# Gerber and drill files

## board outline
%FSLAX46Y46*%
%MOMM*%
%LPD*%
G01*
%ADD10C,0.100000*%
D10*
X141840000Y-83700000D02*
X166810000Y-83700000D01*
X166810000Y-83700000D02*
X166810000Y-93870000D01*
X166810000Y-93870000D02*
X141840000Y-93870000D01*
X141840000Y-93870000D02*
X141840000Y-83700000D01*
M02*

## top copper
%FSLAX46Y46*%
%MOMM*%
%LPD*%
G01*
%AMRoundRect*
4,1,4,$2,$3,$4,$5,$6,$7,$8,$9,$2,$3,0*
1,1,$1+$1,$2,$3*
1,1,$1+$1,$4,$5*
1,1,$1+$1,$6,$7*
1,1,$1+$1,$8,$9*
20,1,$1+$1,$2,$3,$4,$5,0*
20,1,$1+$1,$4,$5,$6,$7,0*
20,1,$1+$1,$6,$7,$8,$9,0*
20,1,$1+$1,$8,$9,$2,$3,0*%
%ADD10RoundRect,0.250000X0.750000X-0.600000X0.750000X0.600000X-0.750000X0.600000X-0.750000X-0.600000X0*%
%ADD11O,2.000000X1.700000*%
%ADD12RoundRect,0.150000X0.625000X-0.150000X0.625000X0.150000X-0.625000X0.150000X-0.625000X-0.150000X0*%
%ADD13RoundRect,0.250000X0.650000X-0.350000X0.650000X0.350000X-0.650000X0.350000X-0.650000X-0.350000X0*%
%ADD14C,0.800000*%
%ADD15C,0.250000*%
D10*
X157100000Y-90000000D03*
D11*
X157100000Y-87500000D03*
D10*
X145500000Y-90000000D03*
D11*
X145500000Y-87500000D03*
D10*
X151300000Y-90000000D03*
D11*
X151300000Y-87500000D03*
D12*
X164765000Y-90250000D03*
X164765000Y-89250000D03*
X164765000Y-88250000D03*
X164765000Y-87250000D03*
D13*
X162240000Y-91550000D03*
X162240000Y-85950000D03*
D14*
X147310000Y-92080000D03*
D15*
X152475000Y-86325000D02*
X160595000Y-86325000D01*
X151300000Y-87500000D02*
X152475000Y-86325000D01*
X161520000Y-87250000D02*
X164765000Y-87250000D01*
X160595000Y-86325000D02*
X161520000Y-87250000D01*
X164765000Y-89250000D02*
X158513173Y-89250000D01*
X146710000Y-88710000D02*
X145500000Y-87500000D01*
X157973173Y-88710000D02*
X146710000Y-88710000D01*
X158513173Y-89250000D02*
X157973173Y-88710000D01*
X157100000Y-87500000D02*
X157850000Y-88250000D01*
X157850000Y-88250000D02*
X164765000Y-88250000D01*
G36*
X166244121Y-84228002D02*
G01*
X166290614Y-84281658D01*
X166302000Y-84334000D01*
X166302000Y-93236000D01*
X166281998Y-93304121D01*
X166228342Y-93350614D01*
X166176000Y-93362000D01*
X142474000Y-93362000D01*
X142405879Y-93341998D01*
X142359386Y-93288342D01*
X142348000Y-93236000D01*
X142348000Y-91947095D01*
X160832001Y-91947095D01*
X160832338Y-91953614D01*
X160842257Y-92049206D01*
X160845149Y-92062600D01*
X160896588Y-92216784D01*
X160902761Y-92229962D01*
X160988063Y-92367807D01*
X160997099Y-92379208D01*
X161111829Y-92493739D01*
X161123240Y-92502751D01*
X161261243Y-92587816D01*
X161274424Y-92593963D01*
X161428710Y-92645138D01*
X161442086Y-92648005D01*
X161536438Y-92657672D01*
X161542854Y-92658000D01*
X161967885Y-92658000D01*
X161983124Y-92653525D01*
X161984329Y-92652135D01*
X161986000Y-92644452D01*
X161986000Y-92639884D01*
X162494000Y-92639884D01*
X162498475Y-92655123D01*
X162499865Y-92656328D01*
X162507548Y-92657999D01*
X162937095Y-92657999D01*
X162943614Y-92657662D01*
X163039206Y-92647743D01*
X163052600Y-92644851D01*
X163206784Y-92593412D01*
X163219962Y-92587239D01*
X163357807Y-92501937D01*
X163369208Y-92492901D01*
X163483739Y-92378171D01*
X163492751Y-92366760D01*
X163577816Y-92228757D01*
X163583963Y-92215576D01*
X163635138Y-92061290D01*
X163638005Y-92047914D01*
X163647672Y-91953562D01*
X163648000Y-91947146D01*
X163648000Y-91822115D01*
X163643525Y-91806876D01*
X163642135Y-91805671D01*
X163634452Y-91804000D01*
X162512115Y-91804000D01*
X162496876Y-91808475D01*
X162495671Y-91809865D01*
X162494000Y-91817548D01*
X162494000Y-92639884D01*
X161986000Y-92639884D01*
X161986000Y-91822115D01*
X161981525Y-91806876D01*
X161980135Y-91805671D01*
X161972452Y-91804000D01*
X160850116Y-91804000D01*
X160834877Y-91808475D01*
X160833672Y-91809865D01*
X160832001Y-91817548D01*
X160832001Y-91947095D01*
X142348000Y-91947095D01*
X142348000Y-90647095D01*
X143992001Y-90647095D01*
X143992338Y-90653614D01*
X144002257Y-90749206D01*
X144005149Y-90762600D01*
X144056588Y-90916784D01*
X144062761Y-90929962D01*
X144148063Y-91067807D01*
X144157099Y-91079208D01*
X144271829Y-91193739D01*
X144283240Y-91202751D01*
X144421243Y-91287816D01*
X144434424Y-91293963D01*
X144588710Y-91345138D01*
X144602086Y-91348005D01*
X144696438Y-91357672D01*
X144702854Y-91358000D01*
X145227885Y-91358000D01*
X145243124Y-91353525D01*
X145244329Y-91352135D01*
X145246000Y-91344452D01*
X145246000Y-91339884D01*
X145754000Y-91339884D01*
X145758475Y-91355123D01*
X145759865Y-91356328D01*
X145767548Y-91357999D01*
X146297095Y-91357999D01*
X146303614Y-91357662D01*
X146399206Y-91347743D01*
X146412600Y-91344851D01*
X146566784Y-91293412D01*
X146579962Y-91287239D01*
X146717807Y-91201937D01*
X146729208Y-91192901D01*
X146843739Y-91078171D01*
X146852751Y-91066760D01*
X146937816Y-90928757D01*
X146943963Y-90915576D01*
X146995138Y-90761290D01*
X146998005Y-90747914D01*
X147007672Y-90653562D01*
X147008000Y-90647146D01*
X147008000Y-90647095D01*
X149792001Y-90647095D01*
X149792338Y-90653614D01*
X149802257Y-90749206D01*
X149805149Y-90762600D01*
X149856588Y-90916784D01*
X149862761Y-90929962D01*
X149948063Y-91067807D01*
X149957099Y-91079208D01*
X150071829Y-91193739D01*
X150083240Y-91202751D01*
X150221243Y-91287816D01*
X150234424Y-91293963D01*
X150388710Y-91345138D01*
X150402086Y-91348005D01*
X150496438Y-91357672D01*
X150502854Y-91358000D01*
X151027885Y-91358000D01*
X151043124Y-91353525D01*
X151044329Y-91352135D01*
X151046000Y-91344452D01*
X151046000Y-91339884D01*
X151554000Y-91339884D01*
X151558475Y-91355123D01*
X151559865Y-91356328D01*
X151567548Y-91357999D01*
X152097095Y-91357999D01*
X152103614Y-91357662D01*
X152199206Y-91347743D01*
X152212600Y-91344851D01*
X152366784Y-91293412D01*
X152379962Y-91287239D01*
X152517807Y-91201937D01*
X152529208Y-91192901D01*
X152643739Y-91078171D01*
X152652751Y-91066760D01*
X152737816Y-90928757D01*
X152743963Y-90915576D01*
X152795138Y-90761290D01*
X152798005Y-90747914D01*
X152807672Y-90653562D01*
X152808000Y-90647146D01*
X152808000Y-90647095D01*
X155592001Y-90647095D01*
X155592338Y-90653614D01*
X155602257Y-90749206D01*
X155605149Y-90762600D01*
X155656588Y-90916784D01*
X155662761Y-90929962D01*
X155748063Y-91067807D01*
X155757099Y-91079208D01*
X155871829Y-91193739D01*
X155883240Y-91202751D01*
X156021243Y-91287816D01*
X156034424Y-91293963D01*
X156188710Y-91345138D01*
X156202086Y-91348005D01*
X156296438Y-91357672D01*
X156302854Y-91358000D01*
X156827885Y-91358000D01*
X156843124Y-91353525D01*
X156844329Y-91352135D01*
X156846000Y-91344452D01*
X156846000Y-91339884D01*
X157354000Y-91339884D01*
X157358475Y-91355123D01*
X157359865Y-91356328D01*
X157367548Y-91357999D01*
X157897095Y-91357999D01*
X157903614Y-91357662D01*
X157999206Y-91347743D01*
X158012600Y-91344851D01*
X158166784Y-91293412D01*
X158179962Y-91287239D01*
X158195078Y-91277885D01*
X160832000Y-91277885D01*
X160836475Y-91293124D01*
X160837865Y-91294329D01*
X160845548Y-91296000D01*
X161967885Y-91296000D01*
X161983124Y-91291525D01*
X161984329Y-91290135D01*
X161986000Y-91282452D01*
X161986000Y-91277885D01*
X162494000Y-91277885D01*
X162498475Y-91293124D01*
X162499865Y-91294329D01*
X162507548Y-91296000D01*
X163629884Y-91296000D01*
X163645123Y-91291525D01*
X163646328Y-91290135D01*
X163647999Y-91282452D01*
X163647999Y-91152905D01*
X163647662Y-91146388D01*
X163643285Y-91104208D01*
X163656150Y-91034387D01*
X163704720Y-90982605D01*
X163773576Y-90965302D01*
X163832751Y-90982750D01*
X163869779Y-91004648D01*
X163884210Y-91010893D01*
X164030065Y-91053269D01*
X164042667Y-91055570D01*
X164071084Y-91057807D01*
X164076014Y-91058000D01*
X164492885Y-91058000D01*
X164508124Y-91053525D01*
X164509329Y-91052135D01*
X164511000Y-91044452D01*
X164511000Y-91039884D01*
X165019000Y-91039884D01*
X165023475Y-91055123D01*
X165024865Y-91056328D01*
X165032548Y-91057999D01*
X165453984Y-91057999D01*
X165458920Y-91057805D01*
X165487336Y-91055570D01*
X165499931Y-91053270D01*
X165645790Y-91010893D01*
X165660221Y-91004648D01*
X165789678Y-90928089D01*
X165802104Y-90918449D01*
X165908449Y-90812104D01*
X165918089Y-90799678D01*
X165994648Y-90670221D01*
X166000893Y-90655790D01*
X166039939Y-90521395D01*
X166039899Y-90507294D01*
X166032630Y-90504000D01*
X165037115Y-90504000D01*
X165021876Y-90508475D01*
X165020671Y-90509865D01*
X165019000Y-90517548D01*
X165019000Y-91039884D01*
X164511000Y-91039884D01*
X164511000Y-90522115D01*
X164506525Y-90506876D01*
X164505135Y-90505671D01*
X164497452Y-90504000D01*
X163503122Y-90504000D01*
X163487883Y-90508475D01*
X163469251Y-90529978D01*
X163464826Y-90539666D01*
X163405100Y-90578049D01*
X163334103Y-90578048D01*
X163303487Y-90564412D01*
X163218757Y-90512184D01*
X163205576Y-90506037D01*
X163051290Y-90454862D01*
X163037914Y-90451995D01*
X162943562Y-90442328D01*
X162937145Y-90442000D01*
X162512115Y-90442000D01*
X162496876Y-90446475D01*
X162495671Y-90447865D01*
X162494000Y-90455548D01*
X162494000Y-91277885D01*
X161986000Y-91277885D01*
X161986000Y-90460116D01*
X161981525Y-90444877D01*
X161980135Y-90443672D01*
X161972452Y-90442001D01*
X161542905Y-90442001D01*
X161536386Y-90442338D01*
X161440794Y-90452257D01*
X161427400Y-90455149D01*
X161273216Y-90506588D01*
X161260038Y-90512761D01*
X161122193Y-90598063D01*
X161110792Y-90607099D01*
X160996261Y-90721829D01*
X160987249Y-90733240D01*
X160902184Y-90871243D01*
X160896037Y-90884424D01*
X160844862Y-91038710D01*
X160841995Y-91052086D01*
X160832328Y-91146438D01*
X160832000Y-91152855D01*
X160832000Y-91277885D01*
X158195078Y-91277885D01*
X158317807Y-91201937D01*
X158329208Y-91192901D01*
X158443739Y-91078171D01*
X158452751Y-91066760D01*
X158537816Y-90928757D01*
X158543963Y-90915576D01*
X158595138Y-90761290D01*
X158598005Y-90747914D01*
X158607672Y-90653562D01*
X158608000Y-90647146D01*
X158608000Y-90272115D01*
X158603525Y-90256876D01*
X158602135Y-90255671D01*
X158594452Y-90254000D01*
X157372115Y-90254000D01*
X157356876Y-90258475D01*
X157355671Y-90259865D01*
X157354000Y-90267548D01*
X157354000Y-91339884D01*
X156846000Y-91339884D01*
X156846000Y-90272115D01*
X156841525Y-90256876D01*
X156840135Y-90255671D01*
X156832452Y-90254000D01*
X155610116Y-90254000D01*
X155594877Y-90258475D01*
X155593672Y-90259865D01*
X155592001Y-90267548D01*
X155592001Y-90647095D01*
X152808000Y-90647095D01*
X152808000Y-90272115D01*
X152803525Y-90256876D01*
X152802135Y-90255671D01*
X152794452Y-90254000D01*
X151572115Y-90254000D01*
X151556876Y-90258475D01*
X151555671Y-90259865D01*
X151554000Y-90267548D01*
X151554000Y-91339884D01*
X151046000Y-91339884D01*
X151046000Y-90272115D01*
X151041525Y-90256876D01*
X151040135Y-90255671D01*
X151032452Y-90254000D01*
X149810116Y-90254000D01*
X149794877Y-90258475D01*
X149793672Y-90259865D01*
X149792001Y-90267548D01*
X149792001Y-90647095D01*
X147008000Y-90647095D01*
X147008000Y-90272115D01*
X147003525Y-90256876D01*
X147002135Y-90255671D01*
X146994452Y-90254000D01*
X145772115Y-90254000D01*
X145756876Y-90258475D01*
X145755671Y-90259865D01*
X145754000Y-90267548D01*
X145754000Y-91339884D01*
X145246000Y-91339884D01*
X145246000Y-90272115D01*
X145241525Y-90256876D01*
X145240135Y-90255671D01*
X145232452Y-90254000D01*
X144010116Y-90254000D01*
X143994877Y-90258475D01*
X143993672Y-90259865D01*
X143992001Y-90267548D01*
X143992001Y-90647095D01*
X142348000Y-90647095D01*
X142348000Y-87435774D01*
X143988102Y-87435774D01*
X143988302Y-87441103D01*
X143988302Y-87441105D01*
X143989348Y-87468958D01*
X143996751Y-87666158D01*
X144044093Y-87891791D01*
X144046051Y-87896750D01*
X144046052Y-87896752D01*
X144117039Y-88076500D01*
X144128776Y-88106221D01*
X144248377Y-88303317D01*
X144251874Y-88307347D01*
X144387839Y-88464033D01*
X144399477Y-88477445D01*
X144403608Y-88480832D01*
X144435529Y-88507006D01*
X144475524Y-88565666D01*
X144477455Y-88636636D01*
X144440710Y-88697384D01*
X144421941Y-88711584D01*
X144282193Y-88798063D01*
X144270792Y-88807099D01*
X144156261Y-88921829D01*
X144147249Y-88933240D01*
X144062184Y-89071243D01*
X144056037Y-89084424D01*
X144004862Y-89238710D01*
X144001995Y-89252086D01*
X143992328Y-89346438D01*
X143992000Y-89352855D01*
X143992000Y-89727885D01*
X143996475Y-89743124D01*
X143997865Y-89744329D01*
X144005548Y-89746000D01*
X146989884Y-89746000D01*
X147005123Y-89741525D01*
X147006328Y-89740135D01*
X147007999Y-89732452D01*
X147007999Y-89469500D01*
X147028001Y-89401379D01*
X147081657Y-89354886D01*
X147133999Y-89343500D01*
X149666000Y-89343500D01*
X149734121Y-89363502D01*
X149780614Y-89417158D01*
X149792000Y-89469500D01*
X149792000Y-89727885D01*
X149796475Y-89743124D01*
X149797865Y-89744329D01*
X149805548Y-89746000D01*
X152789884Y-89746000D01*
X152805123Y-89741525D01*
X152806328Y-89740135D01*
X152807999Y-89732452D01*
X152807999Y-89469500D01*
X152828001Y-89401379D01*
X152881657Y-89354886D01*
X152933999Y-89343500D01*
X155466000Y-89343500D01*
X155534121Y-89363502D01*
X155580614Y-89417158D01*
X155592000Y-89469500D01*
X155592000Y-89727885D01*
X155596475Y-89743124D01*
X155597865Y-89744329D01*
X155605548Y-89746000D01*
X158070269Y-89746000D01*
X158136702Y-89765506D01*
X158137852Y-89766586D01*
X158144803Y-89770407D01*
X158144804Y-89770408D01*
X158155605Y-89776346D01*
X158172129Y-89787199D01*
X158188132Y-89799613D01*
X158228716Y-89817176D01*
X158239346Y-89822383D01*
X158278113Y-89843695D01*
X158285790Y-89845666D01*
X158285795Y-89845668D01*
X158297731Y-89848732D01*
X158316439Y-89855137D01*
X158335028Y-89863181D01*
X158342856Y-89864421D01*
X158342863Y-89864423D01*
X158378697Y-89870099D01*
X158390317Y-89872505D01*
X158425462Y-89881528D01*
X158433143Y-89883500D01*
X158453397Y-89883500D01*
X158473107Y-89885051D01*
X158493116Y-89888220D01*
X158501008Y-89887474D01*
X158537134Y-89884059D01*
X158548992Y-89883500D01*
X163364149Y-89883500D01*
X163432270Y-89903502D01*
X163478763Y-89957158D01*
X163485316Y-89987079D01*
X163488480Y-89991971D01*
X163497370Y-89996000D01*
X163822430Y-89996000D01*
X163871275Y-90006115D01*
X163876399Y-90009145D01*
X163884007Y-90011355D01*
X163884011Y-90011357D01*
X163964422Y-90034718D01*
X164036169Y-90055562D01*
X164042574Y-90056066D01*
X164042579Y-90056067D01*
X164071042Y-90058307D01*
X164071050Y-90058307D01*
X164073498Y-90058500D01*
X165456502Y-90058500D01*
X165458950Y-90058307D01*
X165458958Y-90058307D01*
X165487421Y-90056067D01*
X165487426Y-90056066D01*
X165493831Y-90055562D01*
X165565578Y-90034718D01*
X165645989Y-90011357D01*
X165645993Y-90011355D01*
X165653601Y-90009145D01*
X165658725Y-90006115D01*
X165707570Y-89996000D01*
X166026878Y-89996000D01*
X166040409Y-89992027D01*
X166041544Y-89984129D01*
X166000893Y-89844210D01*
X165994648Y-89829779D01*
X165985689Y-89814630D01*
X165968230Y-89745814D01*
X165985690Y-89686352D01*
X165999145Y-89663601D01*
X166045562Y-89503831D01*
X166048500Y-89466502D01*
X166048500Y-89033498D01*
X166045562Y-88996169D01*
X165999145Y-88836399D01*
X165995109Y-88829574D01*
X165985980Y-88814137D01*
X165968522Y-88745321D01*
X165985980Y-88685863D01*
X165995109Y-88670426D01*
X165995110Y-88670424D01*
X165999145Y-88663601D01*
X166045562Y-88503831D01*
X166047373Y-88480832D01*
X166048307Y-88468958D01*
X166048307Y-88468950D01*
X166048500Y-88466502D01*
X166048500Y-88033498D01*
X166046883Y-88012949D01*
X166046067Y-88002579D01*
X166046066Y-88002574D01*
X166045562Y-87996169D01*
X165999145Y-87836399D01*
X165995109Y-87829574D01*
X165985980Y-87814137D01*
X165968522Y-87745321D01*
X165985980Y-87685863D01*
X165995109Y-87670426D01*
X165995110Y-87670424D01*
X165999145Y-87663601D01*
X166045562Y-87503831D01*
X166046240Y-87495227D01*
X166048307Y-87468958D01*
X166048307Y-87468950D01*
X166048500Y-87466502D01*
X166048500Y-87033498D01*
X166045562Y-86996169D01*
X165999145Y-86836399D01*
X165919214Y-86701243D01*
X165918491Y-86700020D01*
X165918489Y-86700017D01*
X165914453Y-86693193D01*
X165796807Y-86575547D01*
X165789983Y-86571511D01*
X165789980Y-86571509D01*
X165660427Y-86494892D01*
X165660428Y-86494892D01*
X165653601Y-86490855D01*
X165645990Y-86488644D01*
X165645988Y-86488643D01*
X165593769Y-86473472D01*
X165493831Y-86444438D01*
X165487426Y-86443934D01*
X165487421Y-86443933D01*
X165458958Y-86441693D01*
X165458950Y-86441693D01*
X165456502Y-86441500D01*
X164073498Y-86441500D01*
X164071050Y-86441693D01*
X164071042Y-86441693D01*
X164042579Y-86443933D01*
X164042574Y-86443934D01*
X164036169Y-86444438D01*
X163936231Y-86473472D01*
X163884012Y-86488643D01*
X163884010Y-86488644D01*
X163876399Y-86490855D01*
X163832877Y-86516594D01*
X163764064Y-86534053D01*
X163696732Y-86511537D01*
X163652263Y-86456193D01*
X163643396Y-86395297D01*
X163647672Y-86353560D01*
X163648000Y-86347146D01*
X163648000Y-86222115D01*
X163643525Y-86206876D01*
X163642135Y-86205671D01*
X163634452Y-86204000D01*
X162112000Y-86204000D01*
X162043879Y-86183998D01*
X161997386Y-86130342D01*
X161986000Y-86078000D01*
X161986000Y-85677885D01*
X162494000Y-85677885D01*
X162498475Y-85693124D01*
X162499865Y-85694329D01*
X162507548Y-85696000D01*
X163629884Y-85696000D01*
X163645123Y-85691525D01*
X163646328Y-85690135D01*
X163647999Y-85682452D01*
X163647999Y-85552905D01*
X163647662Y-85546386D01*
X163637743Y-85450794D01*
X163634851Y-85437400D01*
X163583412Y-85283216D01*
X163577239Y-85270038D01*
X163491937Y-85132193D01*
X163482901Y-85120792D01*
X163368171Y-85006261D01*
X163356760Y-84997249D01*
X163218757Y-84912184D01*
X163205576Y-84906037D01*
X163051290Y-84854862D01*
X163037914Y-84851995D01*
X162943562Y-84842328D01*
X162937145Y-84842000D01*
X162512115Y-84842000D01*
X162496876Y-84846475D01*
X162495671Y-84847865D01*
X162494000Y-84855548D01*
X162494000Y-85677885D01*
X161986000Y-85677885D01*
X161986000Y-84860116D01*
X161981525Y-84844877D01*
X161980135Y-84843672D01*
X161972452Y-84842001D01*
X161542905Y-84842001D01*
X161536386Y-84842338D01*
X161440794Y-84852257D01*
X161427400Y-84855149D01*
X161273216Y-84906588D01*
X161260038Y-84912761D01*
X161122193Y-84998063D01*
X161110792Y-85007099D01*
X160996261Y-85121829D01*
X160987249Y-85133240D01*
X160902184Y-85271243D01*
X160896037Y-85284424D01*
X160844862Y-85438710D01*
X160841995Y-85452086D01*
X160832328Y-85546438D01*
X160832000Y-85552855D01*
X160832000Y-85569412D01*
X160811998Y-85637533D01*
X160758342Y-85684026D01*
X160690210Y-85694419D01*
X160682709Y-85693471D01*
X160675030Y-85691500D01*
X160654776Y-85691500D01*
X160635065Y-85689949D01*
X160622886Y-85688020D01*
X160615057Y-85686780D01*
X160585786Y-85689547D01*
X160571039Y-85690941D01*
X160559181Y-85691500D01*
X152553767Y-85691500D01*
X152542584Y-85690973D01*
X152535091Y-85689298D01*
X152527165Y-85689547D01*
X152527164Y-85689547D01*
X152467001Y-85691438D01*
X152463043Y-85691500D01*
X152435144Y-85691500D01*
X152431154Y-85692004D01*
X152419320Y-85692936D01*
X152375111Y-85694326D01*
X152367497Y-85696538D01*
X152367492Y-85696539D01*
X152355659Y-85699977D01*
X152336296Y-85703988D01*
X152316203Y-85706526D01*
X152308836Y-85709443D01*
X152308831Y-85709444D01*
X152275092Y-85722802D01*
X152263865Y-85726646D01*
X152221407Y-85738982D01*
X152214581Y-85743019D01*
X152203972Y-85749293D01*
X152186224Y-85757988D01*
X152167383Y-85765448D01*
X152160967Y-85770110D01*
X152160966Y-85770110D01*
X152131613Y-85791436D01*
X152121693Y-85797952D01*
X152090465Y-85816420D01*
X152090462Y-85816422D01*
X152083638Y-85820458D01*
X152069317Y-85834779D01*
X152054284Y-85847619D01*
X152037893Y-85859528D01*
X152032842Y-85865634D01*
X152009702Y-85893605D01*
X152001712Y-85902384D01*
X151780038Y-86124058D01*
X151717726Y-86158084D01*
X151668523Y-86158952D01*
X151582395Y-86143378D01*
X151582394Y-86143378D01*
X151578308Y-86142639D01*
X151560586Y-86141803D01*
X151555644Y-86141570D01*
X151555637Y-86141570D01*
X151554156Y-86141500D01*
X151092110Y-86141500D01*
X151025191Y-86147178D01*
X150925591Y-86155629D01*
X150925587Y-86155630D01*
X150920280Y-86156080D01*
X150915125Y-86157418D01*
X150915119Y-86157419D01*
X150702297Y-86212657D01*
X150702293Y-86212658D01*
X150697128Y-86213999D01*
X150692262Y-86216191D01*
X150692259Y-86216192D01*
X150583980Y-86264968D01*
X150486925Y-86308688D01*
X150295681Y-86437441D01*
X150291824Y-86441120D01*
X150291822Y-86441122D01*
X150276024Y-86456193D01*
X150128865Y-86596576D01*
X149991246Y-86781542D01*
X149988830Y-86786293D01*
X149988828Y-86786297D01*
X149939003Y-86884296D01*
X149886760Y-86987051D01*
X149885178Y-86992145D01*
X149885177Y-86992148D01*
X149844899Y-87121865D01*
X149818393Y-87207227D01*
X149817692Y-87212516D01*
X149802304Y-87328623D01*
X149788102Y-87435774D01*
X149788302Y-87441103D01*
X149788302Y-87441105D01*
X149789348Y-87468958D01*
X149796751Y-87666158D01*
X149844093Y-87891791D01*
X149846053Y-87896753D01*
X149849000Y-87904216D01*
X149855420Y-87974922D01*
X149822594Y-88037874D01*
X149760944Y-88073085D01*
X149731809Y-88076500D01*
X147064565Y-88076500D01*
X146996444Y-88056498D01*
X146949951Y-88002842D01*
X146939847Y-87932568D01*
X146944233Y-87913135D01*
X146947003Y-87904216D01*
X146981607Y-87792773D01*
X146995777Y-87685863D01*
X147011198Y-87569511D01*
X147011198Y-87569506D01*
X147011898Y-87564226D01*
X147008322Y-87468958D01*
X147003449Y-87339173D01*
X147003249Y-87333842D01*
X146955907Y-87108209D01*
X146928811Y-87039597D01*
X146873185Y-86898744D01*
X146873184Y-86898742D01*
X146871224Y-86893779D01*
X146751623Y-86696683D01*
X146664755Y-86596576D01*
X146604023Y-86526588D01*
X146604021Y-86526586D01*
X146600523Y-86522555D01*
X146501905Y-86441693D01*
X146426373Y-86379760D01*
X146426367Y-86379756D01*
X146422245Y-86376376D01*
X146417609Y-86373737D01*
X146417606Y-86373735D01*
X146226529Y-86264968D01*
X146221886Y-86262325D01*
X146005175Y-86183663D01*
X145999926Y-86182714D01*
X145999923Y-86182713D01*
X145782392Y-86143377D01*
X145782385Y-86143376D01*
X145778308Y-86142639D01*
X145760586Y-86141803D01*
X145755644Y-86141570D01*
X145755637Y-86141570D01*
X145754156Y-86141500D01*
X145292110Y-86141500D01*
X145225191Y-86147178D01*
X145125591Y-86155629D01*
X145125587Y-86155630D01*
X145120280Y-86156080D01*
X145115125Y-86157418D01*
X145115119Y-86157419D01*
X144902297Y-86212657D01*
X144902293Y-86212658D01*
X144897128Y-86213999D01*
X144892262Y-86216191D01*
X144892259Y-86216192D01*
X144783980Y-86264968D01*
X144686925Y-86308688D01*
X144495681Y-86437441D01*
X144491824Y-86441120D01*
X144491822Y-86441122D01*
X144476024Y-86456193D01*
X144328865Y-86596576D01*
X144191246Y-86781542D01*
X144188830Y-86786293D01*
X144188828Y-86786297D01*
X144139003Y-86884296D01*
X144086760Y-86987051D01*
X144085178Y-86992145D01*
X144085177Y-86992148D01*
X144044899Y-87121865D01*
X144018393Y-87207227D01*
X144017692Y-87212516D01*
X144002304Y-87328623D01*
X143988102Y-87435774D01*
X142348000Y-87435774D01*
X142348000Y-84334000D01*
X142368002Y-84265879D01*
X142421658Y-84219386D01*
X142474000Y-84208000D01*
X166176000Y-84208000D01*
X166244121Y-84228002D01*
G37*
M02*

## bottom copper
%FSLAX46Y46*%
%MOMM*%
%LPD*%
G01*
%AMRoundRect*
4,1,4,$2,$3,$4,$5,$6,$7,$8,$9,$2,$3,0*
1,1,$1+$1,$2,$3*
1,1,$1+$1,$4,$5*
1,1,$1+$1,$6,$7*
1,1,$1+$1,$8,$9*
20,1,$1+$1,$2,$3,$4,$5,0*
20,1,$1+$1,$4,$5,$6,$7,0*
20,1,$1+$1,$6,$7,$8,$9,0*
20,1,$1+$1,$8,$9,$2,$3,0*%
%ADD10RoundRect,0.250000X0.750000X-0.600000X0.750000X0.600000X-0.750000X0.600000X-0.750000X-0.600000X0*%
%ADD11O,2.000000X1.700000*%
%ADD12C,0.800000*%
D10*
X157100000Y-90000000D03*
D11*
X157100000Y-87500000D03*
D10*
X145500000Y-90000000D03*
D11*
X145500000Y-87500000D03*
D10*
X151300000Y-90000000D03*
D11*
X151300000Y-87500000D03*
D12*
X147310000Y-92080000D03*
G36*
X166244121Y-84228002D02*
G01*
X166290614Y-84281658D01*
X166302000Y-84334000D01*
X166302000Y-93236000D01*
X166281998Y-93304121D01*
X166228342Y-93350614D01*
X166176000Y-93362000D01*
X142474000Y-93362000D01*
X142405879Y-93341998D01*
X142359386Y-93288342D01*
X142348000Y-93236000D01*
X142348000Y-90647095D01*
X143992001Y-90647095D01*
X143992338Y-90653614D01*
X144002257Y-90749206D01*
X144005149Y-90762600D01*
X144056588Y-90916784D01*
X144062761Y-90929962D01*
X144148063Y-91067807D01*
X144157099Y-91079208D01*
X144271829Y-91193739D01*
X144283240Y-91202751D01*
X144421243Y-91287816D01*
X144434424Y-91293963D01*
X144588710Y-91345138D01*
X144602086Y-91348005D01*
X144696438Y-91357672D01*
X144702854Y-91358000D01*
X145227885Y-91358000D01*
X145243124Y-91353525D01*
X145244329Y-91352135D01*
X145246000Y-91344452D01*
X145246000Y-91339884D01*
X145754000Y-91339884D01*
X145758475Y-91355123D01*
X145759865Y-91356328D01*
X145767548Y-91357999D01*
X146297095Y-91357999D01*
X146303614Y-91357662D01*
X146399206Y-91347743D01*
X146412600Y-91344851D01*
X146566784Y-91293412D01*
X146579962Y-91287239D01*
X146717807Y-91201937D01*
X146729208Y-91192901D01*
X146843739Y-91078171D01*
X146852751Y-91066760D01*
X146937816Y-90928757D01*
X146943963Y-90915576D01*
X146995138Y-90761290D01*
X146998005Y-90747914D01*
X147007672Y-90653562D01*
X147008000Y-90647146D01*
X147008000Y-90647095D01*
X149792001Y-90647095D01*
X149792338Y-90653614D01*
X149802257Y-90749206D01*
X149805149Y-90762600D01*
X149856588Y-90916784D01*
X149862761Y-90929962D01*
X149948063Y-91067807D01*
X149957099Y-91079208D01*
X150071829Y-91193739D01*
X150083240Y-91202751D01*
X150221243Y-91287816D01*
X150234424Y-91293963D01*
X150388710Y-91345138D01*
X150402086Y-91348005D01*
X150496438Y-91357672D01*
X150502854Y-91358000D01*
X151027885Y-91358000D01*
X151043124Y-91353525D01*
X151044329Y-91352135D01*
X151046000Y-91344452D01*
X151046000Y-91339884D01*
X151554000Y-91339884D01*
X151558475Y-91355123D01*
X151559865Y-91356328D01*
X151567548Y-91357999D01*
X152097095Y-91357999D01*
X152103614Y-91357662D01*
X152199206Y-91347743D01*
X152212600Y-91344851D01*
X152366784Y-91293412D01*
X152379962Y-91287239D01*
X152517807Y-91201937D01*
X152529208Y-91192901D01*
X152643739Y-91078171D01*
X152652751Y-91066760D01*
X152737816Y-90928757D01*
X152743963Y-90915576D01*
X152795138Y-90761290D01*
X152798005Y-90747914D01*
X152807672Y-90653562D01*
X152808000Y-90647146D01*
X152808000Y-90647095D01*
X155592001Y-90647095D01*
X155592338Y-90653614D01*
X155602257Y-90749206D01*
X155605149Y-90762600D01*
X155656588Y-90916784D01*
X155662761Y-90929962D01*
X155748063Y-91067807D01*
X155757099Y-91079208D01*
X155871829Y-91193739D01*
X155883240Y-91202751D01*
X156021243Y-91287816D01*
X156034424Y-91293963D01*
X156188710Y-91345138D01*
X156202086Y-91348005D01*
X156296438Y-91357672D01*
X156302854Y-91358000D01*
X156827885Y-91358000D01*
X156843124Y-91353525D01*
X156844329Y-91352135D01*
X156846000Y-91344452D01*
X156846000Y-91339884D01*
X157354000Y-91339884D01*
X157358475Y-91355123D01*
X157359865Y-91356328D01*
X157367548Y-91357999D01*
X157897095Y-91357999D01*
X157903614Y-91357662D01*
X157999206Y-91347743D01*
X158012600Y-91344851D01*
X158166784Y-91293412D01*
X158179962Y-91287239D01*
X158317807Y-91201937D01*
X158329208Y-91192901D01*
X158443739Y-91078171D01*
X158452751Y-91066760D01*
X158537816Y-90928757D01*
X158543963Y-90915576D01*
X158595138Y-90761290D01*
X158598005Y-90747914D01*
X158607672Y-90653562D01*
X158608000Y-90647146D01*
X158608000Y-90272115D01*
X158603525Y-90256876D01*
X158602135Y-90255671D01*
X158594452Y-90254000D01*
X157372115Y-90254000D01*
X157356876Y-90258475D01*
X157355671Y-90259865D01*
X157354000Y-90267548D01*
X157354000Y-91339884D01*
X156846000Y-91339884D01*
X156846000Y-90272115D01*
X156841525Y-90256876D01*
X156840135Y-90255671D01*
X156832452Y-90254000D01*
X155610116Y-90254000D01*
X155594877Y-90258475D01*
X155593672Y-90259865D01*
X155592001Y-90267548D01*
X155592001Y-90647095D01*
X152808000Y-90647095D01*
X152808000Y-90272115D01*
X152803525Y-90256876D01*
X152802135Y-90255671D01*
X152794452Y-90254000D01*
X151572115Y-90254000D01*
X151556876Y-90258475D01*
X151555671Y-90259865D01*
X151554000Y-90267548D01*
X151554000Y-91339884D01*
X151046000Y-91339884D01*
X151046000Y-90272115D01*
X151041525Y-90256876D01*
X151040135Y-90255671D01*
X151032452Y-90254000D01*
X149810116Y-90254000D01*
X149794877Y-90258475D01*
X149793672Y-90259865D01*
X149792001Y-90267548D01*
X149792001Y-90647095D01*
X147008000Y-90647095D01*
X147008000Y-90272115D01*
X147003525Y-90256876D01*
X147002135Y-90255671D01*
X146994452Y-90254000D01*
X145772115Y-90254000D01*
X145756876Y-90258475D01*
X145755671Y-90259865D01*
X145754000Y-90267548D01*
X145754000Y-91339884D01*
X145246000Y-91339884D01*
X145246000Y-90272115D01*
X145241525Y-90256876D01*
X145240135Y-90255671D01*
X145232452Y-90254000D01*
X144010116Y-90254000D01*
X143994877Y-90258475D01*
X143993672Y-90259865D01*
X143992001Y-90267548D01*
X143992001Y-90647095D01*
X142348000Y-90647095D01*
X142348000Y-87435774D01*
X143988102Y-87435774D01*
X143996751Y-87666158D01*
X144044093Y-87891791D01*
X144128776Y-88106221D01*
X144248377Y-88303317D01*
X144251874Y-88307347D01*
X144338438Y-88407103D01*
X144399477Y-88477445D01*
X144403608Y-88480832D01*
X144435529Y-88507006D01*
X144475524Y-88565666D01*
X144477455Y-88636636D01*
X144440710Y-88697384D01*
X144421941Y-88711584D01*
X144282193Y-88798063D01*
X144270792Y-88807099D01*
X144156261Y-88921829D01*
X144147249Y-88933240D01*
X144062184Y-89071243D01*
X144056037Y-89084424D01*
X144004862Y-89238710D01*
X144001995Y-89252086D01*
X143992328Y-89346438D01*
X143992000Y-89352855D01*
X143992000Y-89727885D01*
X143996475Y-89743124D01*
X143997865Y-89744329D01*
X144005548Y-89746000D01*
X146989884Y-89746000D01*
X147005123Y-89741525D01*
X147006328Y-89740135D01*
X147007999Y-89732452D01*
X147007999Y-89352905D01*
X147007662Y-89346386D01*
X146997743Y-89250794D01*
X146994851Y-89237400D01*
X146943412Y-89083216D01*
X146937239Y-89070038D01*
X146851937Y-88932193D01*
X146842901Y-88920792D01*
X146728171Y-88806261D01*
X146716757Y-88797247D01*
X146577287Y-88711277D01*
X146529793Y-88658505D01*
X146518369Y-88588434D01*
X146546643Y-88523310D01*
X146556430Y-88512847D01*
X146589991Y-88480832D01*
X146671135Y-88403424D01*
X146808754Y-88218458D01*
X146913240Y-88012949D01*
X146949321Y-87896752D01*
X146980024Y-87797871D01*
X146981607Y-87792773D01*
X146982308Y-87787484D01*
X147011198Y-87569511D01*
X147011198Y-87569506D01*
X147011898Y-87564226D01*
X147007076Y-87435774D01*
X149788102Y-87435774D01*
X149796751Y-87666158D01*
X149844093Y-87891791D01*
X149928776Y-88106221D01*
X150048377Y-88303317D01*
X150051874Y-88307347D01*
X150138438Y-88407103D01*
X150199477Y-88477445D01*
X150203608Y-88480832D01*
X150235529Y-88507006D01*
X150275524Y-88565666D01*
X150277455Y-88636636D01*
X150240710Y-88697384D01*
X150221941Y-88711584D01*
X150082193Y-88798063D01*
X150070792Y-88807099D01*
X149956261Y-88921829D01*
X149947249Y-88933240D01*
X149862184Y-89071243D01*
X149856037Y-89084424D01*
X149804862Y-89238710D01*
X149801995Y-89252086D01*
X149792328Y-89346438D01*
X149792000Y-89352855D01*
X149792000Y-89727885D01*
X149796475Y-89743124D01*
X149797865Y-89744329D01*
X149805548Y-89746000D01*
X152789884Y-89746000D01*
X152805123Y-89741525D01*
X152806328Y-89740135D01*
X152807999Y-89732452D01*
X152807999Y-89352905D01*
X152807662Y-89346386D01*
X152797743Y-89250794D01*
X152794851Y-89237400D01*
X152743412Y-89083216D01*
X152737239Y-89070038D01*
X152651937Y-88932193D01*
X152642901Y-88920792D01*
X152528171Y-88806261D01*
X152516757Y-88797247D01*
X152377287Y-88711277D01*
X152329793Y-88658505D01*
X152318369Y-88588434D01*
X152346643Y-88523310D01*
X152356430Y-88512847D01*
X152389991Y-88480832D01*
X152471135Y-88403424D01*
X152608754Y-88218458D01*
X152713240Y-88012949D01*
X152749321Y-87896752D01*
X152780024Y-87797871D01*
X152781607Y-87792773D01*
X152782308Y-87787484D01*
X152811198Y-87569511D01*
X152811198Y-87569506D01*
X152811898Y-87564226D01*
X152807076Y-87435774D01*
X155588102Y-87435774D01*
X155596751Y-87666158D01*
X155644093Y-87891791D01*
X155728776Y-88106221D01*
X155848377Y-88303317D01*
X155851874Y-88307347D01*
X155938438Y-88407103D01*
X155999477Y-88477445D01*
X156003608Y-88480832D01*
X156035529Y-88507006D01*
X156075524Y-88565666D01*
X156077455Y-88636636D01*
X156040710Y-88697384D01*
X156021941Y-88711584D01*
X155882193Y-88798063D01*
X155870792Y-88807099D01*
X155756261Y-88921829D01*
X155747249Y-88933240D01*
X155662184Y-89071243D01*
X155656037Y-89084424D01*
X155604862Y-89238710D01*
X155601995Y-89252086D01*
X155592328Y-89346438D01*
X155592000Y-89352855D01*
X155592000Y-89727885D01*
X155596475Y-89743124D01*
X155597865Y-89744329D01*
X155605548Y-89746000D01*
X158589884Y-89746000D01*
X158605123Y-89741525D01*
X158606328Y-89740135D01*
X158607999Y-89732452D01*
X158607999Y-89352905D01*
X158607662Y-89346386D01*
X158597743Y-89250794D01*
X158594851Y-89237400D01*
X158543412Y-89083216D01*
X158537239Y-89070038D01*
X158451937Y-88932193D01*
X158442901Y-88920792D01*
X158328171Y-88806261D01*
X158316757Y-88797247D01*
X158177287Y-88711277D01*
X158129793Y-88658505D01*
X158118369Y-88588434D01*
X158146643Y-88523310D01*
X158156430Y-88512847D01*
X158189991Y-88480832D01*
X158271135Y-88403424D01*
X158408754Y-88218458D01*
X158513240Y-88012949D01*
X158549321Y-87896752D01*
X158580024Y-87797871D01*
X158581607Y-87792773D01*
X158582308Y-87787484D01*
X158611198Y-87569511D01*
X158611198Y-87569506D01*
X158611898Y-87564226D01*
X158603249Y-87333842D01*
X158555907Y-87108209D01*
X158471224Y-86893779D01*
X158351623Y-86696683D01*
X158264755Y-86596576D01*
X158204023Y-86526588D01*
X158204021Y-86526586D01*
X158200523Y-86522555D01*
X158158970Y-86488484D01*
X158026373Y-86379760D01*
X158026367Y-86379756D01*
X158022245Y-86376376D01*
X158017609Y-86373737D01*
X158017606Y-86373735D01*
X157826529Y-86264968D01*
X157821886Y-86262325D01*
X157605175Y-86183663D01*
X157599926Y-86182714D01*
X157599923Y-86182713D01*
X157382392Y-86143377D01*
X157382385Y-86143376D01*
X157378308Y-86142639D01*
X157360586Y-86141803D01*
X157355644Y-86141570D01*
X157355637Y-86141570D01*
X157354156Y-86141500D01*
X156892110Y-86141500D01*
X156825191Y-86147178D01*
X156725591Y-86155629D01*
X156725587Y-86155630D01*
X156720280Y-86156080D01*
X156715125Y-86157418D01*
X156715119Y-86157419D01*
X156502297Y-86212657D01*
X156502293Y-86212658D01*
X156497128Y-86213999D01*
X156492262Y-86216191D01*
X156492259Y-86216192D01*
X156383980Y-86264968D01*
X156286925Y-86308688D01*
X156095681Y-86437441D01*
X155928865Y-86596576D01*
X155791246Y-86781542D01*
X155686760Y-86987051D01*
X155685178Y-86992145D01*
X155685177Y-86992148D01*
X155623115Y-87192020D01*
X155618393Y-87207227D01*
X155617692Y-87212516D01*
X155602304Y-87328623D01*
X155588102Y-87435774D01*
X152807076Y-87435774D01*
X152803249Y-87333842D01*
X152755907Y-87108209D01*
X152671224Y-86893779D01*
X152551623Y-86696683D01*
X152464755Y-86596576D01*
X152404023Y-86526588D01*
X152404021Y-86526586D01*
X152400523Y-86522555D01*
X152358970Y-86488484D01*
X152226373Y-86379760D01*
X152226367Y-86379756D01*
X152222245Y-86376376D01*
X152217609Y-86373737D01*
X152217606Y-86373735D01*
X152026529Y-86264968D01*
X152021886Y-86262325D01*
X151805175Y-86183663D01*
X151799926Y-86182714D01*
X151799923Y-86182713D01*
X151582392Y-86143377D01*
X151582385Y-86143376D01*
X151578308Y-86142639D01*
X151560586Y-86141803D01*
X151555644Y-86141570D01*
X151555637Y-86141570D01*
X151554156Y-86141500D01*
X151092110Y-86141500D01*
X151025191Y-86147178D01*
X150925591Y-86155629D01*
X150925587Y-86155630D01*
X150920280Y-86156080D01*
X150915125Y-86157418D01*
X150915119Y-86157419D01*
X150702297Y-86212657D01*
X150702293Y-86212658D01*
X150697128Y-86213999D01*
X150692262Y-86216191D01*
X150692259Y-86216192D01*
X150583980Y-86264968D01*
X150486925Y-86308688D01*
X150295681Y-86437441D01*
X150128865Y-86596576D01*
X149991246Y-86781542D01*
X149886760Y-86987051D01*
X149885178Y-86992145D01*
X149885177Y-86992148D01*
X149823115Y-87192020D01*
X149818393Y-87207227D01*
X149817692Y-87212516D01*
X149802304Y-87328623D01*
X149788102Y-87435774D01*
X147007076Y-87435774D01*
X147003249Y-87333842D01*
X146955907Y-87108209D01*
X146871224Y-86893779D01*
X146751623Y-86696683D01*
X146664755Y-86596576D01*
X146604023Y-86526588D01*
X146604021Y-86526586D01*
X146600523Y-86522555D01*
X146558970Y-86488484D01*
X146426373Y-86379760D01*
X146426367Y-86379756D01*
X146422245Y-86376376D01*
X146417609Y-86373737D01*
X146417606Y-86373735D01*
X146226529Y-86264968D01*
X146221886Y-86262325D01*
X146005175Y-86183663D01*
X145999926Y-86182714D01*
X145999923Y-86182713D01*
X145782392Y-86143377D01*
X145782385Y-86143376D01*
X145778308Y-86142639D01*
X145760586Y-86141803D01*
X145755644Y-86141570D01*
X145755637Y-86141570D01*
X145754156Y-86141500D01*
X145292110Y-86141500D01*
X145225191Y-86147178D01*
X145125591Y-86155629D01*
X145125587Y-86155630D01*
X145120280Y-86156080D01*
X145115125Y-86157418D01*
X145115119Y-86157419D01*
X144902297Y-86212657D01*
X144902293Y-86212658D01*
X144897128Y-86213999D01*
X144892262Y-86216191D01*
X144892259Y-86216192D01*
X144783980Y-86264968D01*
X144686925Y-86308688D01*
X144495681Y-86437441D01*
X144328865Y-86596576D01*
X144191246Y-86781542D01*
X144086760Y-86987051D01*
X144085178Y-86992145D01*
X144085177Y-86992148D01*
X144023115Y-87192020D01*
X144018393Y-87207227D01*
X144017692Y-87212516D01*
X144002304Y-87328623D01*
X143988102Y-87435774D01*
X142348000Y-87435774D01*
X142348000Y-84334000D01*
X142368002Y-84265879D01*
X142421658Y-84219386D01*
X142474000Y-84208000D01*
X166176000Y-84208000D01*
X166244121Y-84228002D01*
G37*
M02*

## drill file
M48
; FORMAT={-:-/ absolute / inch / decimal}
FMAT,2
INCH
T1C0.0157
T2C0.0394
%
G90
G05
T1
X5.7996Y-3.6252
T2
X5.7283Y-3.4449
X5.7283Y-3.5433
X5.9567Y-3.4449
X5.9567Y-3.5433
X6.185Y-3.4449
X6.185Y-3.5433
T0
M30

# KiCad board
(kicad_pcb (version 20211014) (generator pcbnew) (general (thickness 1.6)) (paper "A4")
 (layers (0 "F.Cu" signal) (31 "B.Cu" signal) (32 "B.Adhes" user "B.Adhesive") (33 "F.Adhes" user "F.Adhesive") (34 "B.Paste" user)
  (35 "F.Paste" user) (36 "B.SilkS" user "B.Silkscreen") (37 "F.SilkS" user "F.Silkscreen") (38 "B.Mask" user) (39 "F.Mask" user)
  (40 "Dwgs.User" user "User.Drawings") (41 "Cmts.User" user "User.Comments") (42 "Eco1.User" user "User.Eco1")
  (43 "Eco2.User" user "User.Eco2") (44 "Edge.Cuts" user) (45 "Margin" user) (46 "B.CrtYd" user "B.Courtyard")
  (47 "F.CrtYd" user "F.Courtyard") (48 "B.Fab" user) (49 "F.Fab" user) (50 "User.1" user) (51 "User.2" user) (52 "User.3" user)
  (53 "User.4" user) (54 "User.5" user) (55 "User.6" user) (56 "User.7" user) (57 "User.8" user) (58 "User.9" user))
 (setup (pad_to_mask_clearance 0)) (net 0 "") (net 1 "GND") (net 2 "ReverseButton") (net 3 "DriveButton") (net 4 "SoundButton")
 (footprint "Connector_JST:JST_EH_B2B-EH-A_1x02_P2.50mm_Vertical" (layer "F.Cu") (at 157.1 90 90)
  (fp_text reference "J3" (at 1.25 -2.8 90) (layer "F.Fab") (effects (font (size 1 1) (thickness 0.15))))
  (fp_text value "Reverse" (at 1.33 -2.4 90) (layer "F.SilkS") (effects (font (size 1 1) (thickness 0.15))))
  (pad "1" thru_hole roundrect (at 0 0 90) (size 1.7 2) (drill 1) (layers *.Cu *.Mask) (roundrect_rratio 0.1470588235) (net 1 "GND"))
  (pad "2" thru_hole oval (at 2.5 0 90) (size 1.7 2) (drill 1) (layers *.Cu *.Mask) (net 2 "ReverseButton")))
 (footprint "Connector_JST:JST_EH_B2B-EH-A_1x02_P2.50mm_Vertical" (layer "F.Cu") (at 145.5 90 90)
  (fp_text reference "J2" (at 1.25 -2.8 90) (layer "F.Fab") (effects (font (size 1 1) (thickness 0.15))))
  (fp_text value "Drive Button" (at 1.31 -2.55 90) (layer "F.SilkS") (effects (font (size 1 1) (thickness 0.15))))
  (pad "1" thru_hole roundrect (at 0 0 90) (size 1.7 2) (drill 1) (layers *.Cu *.Mask) (roundrect_rratio 0.1470588235) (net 1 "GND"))
  (pad "2" thru_hole oval (at 2.5 0 90) (size 1.7 2) (drill 1) (layers *.Cu *.Mask) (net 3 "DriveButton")))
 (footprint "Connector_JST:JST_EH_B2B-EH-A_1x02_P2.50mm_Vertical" (layer "F.Cu") (at 151.3 90 90)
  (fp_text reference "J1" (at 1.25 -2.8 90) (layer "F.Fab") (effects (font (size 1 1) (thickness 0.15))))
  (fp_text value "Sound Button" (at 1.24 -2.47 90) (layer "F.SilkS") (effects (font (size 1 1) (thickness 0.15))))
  (pad "1" thru_hole roundrect (at 0 0 90) (size 1.7 2) (drill 1) (layers *.Cu *.Mask) (roundrect_rratio 0.1470588235) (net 1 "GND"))
  (pad "2" thru_hole oval (at 2.5 0 90) (size 1.7 2) (drill 1) (layers *.Cu *.Mask) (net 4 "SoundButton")))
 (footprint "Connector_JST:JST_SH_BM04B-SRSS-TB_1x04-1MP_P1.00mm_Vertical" (layer "F.Cu") (at 163.44 88.75 90)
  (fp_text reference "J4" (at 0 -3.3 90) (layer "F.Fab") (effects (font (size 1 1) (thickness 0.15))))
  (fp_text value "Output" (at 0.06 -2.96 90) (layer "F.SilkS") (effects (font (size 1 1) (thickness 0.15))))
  (pad "1" smd roundrect (at -1.5 1.325 90) (size 0.6 1.55) (layers "F.Cu" "F.Paste" "F.Mask") (roundrect_rratio 0.25) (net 1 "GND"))
  (pad "2" smd roundrect (at -0.5 1.325 90) (size 0.6 1.55) (layers "F.Cu" "F.Paste" "F.Mask") (roundrect_rratio 0.25) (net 3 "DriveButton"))
  (pad "3" smd roundrect (at 0.5 1.325 90) (size 0.6 1.55) (layers "F.Cu" "F.Paste" "F.Mask") (roundrect_rratio 0.25)
   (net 2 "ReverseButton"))
  (pad "4" smd roundrect (at 1.5 1.325 90) (size 0.6 1.55) (layers "F.Cu" "F.Paste" "F.Mask") (roundrect_rratio 0.25) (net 4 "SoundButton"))
  (pad "MP" smd roundrect (at -2.8 -1.2 90) (size 1.2 1.8) (layers "F.Cu" "F.Paste" "F.Mask") (roundrect_rratio 0.2083333333) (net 1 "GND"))
  (pad "MP" smd roundrect (at 2.8 -1.2 90) (size 1.2 1.8) (layers "F.Cu" "F.Paste" "F.Mask") (roundrect_rratio 0.2083333333) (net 1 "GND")))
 (gr_rect (start 141.84 83.7) (end 166.81 93.87) (layer "Edge.Cuts") (width 0.1) (fill none))
 (via (at 147.31 92.08) (size 0.8) (drill 0.4) (layers "F.Cu" "B.Cu") (free) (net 1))
 (segment (start 152.475 86.325) (end 160.595 86.325) (width 0.25) (layer "F.Cu") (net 4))
 (segment (start 151.3 87.5) (end 152.475 86.325) (width 0.25) (layer "F.Cu") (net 4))
 (segment (start 161.52 87.25) (end 164.765 87.25) (width 0.25) (layer "F.Cu") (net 4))
 (segment (start 160.595 86.325) (end 161.52 87.25) (width 0.25) (layer "F.Cu") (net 4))
 (segment (start 164.765 89.25) (end 158.513173 89.25) (width 0.25) (layer "F.Cu") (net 3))
 (segment (start 146.71 88.71) (end 145.5 87.5) (width 0.25) (layer "F.Cu") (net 3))
 (segment (start 157.973173 88.71) (end 146.71 88.71) (width 0.25) (layer "F.Cu") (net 3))
 (segment (start 158.513173 89.25) (end 157.973173 88.71) (width 0.25) (layer "F.Cu") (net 3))
 (segment (start 157.1 87.5) (end 157.85 88.25) (width 0.25) (layer "F.Cu") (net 2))
 (segment (start 157.85 88.25) (end 164.765 88.25) (width 0.25) (layer "F.Cu") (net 2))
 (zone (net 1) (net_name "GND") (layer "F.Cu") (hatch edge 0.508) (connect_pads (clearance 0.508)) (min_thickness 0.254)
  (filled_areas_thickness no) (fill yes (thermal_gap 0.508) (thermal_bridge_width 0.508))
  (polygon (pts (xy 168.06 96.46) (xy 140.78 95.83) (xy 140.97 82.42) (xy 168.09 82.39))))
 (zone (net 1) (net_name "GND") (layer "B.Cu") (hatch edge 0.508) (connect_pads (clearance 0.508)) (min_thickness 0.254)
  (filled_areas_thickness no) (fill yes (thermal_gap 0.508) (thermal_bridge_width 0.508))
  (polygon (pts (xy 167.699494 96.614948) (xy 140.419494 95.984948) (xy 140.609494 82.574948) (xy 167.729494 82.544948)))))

